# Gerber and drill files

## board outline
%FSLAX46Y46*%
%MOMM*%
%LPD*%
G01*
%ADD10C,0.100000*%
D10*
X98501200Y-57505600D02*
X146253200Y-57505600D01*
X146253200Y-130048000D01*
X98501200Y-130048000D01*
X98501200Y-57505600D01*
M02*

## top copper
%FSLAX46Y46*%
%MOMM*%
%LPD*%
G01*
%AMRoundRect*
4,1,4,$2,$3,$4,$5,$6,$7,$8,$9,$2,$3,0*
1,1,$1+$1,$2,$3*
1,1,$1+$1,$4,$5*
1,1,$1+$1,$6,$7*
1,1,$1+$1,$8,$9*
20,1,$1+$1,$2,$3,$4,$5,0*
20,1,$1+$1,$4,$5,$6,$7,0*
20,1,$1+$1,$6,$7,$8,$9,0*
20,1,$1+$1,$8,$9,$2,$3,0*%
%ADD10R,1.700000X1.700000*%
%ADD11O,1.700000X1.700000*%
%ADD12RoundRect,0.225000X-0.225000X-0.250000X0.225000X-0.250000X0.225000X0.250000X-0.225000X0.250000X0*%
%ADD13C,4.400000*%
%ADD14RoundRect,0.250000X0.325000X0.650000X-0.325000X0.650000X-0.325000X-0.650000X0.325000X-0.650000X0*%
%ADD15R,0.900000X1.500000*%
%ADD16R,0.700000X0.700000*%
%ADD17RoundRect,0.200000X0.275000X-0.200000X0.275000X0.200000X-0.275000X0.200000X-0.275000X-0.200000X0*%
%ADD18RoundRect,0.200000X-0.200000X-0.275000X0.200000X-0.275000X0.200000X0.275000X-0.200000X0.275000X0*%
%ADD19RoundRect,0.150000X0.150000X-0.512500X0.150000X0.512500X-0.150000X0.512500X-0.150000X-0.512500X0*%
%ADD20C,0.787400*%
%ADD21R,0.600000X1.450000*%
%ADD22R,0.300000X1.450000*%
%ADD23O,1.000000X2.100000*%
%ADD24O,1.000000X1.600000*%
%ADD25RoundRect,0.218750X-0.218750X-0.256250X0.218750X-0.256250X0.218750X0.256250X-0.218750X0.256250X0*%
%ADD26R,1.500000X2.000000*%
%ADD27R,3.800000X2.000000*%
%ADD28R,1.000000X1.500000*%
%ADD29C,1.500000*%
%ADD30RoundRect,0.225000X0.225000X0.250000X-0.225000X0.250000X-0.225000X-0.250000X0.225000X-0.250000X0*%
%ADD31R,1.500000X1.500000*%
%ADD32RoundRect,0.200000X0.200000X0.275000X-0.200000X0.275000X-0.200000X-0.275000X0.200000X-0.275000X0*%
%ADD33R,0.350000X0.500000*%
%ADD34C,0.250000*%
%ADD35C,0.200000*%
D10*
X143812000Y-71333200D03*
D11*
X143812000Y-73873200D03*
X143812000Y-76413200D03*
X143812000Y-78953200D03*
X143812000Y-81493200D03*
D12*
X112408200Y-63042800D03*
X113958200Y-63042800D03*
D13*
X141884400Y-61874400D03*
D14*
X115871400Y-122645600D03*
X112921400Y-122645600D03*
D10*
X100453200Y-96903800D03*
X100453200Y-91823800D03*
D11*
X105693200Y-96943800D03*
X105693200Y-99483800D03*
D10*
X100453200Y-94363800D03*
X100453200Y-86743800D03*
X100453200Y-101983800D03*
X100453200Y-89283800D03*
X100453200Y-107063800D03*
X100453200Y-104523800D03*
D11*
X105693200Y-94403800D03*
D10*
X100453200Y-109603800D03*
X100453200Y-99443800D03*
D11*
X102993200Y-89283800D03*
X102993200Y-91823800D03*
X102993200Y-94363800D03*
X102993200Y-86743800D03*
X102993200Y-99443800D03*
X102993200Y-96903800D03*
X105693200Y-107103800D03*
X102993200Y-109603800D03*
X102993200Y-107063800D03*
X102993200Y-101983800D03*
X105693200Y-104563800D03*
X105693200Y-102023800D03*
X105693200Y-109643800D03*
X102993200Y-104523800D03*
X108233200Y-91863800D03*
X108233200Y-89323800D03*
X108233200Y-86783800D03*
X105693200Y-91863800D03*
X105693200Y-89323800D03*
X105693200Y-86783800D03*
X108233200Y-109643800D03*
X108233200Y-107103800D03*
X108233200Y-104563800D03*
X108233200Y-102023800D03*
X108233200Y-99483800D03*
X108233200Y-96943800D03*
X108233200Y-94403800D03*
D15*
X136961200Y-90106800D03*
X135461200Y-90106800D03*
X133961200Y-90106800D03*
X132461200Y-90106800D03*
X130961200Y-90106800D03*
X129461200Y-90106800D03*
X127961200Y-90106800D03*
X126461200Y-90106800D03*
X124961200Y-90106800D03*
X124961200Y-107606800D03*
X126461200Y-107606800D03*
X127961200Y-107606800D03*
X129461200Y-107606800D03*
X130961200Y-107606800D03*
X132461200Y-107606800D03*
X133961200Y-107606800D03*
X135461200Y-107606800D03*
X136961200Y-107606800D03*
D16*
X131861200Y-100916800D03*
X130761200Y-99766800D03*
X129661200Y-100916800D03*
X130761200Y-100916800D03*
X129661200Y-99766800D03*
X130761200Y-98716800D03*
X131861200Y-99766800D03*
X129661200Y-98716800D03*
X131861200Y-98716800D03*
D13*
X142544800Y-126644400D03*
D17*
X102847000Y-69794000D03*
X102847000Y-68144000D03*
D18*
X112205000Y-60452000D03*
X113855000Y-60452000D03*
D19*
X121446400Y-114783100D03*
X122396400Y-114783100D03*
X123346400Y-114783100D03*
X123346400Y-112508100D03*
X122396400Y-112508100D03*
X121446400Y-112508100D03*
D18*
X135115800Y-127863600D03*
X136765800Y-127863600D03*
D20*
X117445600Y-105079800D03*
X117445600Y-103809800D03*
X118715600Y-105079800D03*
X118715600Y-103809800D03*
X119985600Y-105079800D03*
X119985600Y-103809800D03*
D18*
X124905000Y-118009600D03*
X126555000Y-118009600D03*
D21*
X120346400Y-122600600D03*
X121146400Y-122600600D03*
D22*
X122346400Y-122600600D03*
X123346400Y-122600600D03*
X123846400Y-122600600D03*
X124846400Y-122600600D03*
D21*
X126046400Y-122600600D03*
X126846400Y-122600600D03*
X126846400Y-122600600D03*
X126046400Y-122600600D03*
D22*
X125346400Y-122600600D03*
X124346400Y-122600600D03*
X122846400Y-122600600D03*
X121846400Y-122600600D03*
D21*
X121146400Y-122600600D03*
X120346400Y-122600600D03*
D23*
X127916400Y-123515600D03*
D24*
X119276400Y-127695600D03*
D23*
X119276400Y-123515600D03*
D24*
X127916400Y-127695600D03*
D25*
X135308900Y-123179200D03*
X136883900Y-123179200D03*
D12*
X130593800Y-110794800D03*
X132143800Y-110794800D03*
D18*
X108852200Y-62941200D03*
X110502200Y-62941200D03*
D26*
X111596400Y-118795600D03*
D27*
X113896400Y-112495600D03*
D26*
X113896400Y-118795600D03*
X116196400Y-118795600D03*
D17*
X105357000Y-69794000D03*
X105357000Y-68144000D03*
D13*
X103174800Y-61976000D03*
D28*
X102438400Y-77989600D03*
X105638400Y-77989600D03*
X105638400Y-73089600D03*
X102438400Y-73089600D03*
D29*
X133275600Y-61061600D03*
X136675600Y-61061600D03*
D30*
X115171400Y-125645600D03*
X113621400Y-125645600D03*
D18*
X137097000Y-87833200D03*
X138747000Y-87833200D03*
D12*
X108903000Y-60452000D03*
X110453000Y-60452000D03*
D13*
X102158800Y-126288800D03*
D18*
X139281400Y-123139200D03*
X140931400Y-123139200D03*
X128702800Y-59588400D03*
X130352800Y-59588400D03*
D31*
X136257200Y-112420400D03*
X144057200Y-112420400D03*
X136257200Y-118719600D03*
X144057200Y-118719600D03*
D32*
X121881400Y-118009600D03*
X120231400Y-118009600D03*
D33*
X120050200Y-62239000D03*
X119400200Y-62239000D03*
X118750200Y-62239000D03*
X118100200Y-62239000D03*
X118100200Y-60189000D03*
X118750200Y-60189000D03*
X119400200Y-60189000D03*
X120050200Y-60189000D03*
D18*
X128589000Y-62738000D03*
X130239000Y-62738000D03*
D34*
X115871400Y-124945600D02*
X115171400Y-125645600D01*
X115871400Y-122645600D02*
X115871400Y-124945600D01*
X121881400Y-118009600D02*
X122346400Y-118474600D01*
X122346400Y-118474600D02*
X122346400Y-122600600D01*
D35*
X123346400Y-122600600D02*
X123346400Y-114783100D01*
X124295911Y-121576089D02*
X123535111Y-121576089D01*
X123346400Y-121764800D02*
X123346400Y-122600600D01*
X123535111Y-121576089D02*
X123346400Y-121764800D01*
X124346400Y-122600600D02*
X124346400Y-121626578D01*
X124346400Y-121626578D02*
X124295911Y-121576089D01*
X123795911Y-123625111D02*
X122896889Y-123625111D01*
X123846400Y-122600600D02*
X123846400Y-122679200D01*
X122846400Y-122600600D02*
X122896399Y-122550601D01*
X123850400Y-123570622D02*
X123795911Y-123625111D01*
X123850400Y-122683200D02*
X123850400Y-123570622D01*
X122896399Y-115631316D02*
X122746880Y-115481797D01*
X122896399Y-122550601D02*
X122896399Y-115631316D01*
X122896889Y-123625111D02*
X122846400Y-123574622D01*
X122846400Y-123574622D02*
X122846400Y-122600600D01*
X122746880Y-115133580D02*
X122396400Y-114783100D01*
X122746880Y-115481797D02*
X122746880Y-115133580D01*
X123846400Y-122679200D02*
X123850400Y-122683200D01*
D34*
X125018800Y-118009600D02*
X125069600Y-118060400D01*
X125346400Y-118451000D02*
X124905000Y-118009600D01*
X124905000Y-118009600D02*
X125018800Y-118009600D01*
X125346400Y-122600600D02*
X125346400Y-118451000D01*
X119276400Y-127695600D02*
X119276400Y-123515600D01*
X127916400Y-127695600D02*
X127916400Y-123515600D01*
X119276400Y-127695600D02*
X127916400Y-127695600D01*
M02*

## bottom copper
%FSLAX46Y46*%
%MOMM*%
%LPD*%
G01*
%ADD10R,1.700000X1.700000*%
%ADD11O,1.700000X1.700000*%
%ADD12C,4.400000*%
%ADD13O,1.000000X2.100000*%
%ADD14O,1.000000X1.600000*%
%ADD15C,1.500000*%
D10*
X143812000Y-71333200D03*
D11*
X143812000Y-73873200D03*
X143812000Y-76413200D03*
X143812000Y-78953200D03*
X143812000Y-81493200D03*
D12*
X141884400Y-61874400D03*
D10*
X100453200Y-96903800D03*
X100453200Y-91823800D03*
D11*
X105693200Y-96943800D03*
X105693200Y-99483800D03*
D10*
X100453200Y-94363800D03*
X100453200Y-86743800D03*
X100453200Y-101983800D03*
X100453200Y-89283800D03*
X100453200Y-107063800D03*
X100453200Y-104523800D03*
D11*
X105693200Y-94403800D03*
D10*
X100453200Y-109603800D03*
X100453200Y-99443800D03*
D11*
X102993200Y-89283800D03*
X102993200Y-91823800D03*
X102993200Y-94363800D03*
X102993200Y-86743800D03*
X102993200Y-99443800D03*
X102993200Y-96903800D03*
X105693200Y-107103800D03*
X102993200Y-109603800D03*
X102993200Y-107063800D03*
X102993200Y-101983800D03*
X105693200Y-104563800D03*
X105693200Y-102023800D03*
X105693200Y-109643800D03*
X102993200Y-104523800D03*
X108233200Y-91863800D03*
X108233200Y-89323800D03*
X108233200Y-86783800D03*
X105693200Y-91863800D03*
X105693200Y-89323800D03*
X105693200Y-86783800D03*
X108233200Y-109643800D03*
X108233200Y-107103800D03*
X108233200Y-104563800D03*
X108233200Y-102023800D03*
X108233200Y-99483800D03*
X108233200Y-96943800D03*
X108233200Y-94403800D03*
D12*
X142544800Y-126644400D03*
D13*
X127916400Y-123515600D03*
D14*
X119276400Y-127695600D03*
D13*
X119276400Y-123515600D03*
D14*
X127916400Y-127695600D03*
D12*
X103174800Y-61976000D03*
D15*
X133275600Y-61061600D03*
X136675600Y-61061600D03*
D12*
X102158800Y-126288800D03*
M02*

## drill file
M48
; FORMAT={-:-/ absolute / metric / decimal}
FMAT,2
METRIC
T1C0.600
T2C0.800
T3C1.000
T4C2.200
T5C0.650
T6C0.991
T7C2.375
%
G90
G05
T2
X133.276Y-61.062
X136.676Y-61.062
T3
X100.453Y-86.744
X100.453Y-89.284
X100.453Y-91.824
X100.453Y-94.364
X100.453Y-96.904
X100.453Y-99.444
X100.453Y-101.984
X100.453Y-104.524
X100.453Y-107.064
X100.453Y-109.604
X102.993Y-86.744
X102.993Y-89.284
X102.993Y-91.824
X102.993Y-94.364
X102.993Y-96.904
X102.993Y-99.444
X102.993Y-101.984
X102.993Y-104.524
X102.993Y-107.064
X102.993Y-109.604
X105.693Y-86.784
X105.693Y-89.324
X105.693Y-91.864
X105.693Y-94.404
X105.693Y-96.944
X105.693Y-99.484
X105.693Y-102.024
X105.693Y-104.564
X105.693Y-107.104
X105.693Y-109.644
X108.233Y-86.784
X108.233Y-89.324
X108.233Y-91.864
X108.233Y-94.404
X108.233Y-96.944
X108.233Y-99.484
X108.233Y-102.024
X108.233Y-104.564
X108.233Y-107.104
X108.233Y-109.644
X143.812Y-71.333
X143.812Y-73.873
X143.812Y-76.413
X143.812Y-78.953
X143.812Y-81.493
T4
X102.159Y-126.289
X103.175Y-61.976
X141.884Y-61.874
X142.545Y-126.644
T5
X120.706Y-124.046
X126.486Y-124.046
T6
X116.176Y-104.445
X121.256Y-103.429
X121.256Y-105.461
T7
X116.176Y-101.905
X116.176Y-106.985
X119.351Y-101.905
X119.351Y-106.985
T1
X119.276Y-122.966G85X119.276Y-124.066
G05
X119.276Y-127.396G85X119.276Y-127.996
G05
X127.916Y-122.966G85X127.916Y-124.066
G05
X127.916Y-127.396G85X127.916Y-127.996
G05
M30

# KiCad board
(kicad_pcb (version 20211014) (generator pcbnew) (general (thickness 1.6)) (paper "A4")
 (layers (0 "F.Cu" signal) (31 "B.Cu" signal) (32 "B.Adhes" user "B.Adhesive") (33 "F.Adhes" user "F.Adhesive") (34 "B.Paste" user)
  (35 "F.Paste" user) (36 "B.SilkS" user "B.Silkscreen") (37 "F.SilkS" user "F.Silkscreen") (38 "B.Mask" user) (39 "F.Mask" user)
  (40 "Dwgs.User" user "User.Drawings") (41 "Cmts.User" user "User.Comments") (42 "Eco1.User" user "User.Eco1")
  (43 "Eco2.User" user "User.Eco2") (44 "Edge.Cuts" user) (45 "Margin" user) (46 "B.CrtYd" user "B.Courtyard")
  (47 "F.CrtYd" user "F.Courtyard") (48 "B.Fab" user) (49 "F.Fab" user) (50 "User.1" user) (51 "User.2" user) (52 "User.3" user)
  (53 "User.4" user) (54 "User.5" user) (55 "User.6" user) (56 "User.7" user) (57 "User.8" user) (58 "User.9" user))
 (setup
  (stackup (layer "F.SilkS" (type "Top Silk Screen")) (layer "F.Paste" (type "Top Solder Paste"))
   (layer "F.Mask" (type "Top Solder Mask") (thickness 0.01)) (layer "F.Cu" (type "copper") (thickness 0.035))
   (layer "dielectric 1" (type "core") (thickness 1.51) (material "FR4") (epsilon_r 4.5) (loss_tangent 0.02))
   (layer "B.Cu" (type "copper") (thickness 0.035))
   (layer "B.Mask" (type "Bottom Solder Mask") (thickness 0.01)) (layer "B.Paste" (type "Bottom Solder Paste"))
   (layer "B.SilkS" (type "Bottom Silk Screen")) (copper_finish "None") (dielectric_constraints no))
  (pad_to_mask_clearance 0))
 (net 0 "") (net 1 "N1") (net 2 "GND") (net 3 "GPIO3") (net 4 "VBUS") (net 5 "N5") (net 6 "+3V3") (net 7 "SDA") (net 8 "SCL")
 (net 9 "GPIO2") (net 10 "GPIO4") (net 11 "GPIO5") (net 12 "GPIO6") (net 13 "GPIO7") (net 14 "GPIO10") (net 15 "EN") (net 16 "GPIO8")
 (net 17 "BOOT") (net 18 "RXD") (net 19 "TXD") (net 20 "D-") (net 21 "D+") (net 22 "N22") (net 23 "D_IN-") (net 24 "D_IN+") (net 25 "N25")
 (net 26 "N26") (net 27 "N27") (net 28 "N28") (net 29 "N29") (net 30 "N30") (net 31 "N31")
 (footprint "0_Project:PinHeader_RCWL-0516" (layer "F.Cu") (at 143.812 71.3332)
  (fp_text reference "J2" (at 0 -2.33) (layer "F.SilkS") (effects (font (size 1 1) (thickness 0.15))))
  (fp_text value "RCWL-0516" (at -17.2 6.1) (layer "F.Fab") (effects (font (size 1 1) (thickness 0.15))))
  (pad "1" thru_hole rect (at 0 0) (size 1.7 1.7) (drill 1) (layers *.Cu *.Mask) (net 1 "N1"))
  (pad "2" thru_hole oval (at 0 2.54) (size 1.7 1.7) (drill 1) (layers *.Cu *.Mask) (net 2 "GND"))
  (pad "3" thru_hole oval (at 0 5.08) (size 1.7 1.7) (drill 1) (layers *.Cu *.Mask) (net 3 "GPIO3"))
  (pad "4" thru_hole oval (at 0 7.62) (size 1.7 1.7) (drill 1) (layers *.Cu *.Mask) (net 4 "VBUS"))
  (pad "5" thru_hole oval (at 0 10.16) (size 1.7 1.7) (drill 1) (layers *.Cu *.Mask) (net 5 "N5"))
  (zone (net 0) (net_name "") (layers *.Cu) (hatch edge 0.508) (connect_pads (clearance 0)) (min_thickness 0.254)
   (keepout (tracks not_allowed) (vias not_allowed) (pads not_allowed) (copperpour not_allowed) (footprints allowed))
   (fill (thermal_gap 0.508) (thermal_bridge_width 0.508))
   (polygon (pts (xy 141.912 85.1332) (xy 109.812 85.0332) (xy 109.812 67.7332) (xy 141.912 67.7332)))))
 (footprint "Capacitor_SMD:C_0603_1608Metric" (layer "F.Cu") (at 113.1832 63.0428)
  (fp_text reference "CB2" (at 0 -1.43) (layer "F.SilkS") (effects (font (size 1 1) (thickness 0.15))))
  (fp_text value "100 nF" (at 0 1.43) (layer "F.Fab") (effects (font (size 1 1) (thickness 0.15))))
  (pad "1" smd roundrect (at -0.775 0) (size 0.9 0.95) (layers "F.Cu" "F.Paste" "F.Mask") (roundrect_rratio 0.25) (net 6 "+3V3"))
  (pad "2" smd roundrect (at 0.775 0) (size 0.9 0.95) (layers "F.Cu" "F.Paste" "F.Mask") (roundrect_rratio 0.25) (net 2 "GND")))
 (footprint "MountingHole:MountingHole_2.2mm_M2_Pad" (layer "F.Cu") (at 141.8844 61.8744)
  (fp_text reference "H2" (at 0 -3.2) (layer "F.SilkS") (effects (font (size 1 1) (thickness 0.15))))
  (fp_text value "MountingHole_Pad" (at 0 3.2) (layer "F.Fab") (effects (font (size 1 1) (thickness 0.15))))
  (pad "1" thru_hole circle (at 0 0) (size 4.4 4.4) (drill 2.2) (layers *.Cu *.Mask) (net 2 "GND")))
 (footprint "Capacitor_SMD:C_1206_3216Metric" (layer "F.Cu") (at 114.3964 122.6456 180)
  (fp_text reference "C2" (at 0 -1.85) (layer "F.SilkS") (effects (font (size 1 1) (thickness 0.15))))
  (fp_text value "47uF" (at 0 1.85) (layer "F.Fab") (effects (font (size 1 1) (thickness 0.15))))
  (pad "1" smd roundrect (at -1.475 0 180) (size 1.15 1.8) (layers "F.Cu" "F.Paste" "F.Mask") (roundrect_rratio 0.217391) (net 4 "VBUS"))
  (pad "2" smd roundrect (at 1.475 0 180) (size 1.15 1.8) (layers "F.Cu" "F.Paste" "F.Mask") (roundrect_rratio 0.217391) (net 2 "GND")))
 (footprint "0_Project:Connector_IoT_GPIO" (layer "F.Cu") (at 106.8932 114.7038 180)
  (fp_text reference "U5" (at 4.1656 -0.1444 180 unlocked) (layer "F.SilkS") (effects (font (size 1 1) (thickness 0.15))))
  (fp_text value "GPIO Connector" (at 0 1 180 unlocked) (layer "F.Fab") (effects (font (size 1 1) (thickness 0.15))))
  (pad "1" thru_hole rect (at 6.44 17.8 180) (size 1.7 1.7) (drill 1) (layers *.Cu *.Mask) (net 2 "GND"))
  (pad "1" thru_hole rect (at 6.44 22.88 180) (size 1.7 1.7) (drill 1) (layers *.Cu *.Mask) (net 2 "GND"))
  (pad "1" thru_hole oval (at 1.2 17.76 180) (size 1.7 1.7) (drill 1) (layers *.Cu *.Mask) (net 2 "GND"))
  (pad "1" thru_hole oval (at 1.2 15.22 180) (size 1.7 1.7) (drill 1) (layers *.Cu *.Mask) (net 2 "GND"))
  (pad "1" thru_hole rect (at 6.44 20.34 180) (size 1.7 1.7) (drill 1) (layers *.Cu *.Mask) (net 2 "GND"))
  (pad "1" thru_hole rect (at 6.44 27.96 180) (size 1.7 1.7) (drill 1) (layers *.Cu *.Mask) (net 2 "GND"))
  (pad "1" thru_hole rect (at 6.44 12.72 180) (size 1.7 1.7) (drill 1) (layers *.Cu *.Mask) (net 2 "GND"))
  (pad "1" thru_hole rect (at 6.44 25.42 180) (size 1.7 1.7) (drill 1) (layers *.Cu *.Mask) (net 2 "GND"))
  (pad "1" thru_hole rect (at 6.44 7.64 180) (size 1.7 1.7) (drill 1) (layers *.Cu *.Mask) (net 2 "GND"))
  (pad "1" thru_hole rect (at 6.44 10.18 180) (size 1.7 1.7) (drill 1) (layers *.Cu *.Mask) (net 2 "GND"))
  (pad "1" thru_hole oval (at 1.2 20.3 180) (size 1.7 1.7) (drill 1) (layers *.Cu *.Mask) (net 2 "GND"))
  (pad "1" thru_hole rect (at 6.44 5.1 180) (size 1.7 1.7) (drill 1) (layers *.Cu *.Mask) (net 2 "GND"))
  (pad "1" thru_hole rect (at 6.44 15.26 180) (size 1.7 1.7) (drill 1) (layers *.Cu *.Mask) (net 2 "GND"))
  (pad "2" thru_hole oval (at 3.9 25.42 180) (size 1.7 1.7) (drill 1) (layers *.Cu *.Mask) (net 6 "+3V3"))
  (pad "2" thru_hole oval (at 3.9 22.88 180) (size 1.7 1.7) (drill 1) (layers *.Cu *.Mask) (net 6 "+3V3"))
  (pad "2" thru_hole oval (at 3.9 20.34 180) (size 1.7 1.7) (drill 1) (layers *.Cu *.Mask) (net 6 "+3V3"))
  (pad "2" thru_hole oval (at 3.9 27.96 180) (size 1.7 1.7) (drill 1) (layers *.Cu *.Mask) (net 6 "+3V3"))
  (pad "2" thru_hole oval (at 3.9 15.26 180) (size 1.7 1.7) (drill 1) (layers *.Cu *.Mask) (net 6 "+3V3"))
  (pad "2" thru_hole oval (at 3.9 17.8 180) (size 1.7 1.7) (drill 1) (layers *.Cu *.Mask) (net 6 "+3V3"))
  (pad "3" thru_hole oval (at 1.2 7.6 180) (size 1.7 1.7) (drill 1) (layers *.Cu *.Mask) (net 4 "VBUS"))
  (pad "3" thru_hole oval (at 3.9 5.1 180) (size 1.7 1.7) (drill 1) (layers *.Cu *.Mask) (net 4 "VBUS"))
  (pad "3" thru_hole oval (at 3.9 7.64 180) (size 1.7 1.7) (drill 1) (layers *.Cu *.Mask) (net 4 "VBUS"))
  (pad "3" thru_hole oval (at 3.9 12.72 180) (size 1.7 1.7) (drill 1) (layers *.Cu *.Mask) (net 4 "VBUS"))
  (pad "3" thru_hole oval (at 1.2 10.14 180) (size 1.7 1.7) (drill 1) (layers *.Cu *.Mask) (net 4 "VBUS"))
  (pad "3" thru_hole oval (at 1.2 12.68 180) (size 1.7 1.7) (drill 1) (layers *.Cu *.Mask) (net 4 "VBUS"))
  (pad "3" thru_hole oval (at 1.2 5.06 180) (size 1.7 1.7) (drill 1) (layers *.Cu *.Mask) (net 4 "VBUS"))
  (pad "3" thru_hole oval (at 3.9 10.18 180) (size 1.7 1.7) (drill 1) (layers *.Cu *.Mask) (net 4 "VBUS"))
  (pad "4" thru_hole oval (at -1.34 22.84 180) (size 1.7 1.7) (drill 1) (layers *.Cu *.Mask) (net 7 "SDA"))
  (pad "4" thru_hole oval (at -1.34 25.38 180) (size 1.7 1.7) (drill 1) (layers *.Cu *.Mask) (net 7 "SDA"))
  (pad "4" thru_hole oval (at -1.34 27.92 180) (size 1.7 1.7) (drill 1) (layers *.Cu *.Mask) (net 7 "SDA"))
  (pad "5" thru_hole oval (at 1.2 22.84 180) (size 1.7 1.7) (drill 1) (layers *.Cu *.Mask) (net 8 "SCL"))
  (pad "5" thru_hole oval (at 1.2 25.38 180) (size 1.7 1.7) (drill 1) (layers *.Cu *.Mask) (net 8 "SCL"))
  (pad "5" thru_hole oval (at 1.2 27.92 180) (size 1.7 1.7) (drill 1) (layers *.Cu *.Mask) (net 8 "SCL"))
  (pad "6" thru_hole oval (at -1.34 5.06 180) (size 1.7 1.7) (drill 1) (layers *.Cu *.Mask) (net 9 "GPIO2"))
  (pad "7" thru_hole oval (at -1.34 7.6 180) (size 1.7 1.7) (drill 1) (layers *.Cu *.Mask) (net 3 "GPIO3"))
  (pad "8" thru_hole oval (at -1.34 10.14 180) (size 1.7 1.7) (drill 1) (layers *.Cu *.Mask) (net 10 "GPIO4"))
  (pad "9" thru_hole oval (at -1.34 12.68 180) (size 1.7 1.7) (drill 1) (layers *.Cu *.Mask) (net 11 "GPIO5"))
  (pad "10" thru_hole oval (at -1.34 15.22 180) (size 1.7 1.7) (drill 1) (layers *.Cu *.Mask) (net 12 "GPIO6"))
  (pad "11" thru_hole oval (at -1.34 17.76 180) (size 1.7 1.7) (drill 1) (layers *.Cu *.Mask) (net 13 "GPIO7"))
  (pad "12" thru_hole oval (at -1.34 20.3 180) (size 1.7 1.7) (drill 1) (layers *.Cu *.Mask) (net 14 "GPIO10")))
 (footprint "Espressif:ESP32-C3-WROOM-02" (layer "F.Cu") (at 132.8112 98.8568 -90)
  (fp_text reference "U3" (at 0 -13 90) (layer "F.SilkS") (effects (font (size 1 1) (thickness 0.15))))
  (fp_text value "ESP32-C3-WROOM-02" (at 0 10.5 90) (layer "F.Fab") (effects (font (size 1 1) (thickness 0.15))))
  (pad "1" smd rect locked (at -8.75 -4.15 270) (size 1.5 0.9) (layers "F.Cu" "F.Paste" "F.Mask") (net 6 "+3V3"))
  (pad "2" smd rect locked (at -8.75 -2.65 270) (size 1.5 0.9) (layers "F.Cu" "F.Paste" "F.Mask") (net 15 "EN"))
  (pad "3" smd rect locked (at -8.75 -1.15 270) (size 1.5 0.9) (layers "F.Cu" "F.Paste" "F.Mask") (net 10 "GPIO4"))
  (pad "4" smd rect locked (at -8.75 0.35 270) (size 1.5 0.9) (layers "F.Cu" "F.Paste" "F.Mask") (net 11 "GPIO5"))
  (pad "5" smd rect locked (at -8.75 1.85 270) (size 1.5 0.9) (layers "F.Cu" "F.Paste" "F.Mask") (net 12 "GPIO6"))
  (pad "6" smd rect locked (at -8.75 3.35 270) (size 1.5 0.9) (layers "F.Cu" "F.Paste" "F.Mask") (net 13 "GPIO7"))
  (pad "7" smd rect locked (at -8.75 4.85 270) (size 1.5 0.9) (layers "F.Cu" "F.Paste" "F.Mask") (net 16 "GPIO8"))
  (pad "8" smd rect locked (at -8.75 6.35 270) (size 1.5 0.9) (layers "F.Cu" "F.Paste" "F.Mask") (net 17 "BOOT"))
  (pad "9" smd rect locked (at -8.75 7.85 270) (size 1.5 0.9) (layers "F.Cu" "F.Paste" "F.Mask") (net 2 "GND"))
  (pad "10" smd rect locked (at 8.75 7.85 90) (size 1.5 0.9) (layers "F.Cu" "F.Paste" "F.Mask") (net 14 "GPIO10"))
  (pad "11" smd rect locked (at 8.75 6.35 90) (size 1.5 0.9) (layers "F.Cu" "F.Paste" "F.Mask") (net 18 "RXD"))
  (pad "12" smd rect locked (at 8.75 4.85 90) (size 1.5 0.9) (layers "F.Cu" "F.Paste" "F.Mask") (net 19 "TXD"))
  (pad "13" smd rect locked (at 8.75 3.35 90) (size 1.5 0.9) (layers "F.Cu" "F.Paste" "F.Mask") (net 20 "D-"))
  (pad "14" smd rect locked (at 8.75 1.85 90) (size 1.5 0.9) (layers "F.Cu" "F.Paste" "F.Mask") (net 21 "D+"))
  (pad "15" smd rect locked (at 8.75 0.35 90) (size 1.5 0.9) (layers "F.Cu" "F.Paste" "F.Mask") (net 3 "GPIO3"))
  (pad "16" smd rect locked (at 8.75 -1.15 90) (size 1.5 0.9) (layers "F.Cu" "F.Paste" "F.Mask") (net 9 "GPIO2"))
  (pad "17" smd rect locked (at 8.75 -2.65 90) (size 1.5 0.9) (layers "F.Cu" "F.Paste" "F.Mask") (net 8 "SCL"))
  (pad "18" smd rect locked (at 8.75 -4.15 90) (size 1.5 0.9) (layers "F.Cu" "F.Paste" "F.Mask") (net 7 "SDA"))
  (pad "19" smd rect locked (at 2.06 0.95 90) (size 0.7 0.7) (layers "F.Cu" "F.Paste" "F.Mask") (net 2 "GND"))
  (pad "19" smd rect locked (at 0.91 2.05 90) (size 0.7 0.7) (layers "F.Cu" "F.Paste" "F.Mask") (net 2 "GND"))
  (pad "19" smd rect locked (at 2.06 3.15 90) (size 0.7 0.7) (layers "F.Cu" "F.Paste" "F.Mask") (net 2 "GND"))
  (pad "19" smd rect locked (at 2.06 2.05 90) (size 0.7 0.7) (layers "F.Cu" "F.Paste" "F.Mask") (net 2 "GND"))
  (pad "19" smd rect locked (at 0.91 3.15 90) (size 0.7 0.7) (layers "F.Cu" "F.Paste" "F.Mask") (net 2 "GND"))
  (pad "19" smd rect locked (at -0.14 2.05 90) (size 0.7 0.7) (layers "F.Cu" "F.Paste" "F.Mask") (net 2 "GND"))
  (pad "19" smd rect locked (at 0.91 0.95 90) (size 0.7 0.7) (layers "F.Cu" "F.Paste" "F.Mask") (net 2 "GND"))
  (pad "19" smd rect locked (at -0.14 3.15 90) (size 0.7 0.7) (layers "F.Cu" "F.Paste" "F.Mask") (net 2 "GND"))
  (pad "19" smd rect locked (at -0.14 0.95 90) (size 0.7 0.7) (layers "F.Cu" "F.Paste" "F.Mask") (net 2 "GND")))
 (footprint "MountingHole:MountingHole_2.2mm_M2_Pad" (layer "F.Cu") (at 142.5448 126.6444)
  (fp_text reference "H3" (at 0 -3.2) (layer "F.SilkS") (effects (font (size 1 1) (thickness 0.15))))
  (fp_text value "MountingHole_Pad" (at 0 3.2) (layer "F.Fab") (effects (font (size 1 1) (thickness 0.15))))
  (pad "1" thru_hole circle (at 0 0) (size 4.4 4.4) (drill 2.2) (layers *.Cu *.Mask) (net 2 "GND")))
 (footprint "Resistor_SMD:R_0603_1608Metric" (layer "F.Cu") (at 102.847 68.969 90)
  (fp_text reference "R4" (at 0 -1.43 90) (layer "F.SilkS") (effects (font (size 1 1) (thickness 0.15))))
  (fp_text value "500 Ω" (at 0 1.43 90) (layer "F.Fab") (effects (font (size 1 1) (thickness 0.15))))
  (pad "1" smd roundrect (at -0.825 0 90) (size 0.8 0.95) (layers "F.Cu" "F.Paste" "F.Mask") (roundrect_rratio 0.25) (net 16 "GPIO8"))
  (pad "2" smd roundrect (at 0.825 0 90) (size 0.8 0.95) (layers "F.Cu" "F.Paste" "F.Mask") (roundrect_rratio 0.25) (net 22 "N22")))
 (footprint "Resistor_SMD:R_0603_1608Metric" (layer "F.Cu") (at 113.03 60.452)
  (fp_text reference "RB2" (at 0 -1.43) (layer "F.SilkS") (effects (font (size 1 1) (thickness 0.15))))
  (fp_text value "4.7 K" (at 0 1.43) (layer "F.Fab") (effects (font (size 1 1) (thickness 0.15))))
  (pad "1" smd roundrect (at -0.825 0) (size 0.8 0.95) (layers "F.Cu" "F.Paste" "F.Mask") (roundrect_rratio 0.25) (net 8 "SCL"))
  (pad "2" smd roundrect (at 0.825 0) (size 0.8 0.95) (layers "F.Cu" "F.Paste" "F.Mask") (roundrect_rratio 0.25) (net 6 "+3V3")))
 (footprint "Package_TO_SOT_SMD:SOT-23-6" (layer "F.Cu") (at 122.3964 113.6456 90)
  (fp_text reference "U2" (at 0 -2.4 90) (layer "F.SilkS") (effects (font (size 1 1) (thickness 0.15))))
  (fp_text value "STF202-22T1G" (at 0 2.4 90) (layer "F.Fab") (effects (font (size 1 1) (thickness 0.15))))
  (pad "1" smd roundrect (at -1.1375 -0.95 90) (size 1.325 0.6) (layers "F.Cu" "F.Paste" "F.Mask") (roundrect_rratio 0.25) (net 4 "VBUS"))
  (pad "2" smd roundrect (at -1.1375 0 90) (size 1.325 0.6) (layers "F.Cu" "F.Paste" "F.Mask") (roundrect_rratio 0.25) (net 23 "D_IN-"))
  (pad "3" smd roundrect (at -1.1375 0.95 90) (size 1.325 0.6) (layers "F.Cu" "F.Paste" "F.Mask") (roundrect_rratio 0.25) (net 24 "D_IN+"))
  (pad "4" smd roundrect (at 1.1375 0.95 90) (size 1.325 0.6) (layers "F.Cu" "F.Paste" "F.Mask") (roundrect_rratio 0.25) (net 21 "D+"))
  (pad "5" smd roundrect (at 1.1375 0 90) (size 1.325 0.6) (layers "F.Cu" "F.Paste" "F.Mask") (roundrect_rratio 0.25) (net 20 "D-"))
  (pad "6" smd roundrect (at 1.1375 -0.95 90) (size 1.325 0.6) (layers "F.Cu" "F.Paste" "F.Mask") (roundrect_rratio 0.25) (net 2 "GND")))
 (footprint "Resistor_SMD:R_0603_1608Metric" (layer "F.Cu") (at 135.9408 127.8636)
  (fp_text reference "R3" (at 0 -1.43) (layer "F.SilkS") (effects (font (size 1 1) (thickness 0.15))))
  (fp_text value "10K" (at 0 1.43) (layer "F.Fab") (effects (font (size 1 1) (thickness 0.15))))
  (pad "1" smd roundrect (at -0.825 0) (size 0.8 0.95) (layers "F.Cu" "F.Paste" "F.Mask") (roundrect_rratio 0.25) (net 6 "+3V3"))
  (pad "2" smd roundrect (at 0.825 0) (size 0.8 0.95) (layers "F.Cu" "F.Paste" "F.Mask") (roundrect_rratio 0.25) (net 15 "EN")))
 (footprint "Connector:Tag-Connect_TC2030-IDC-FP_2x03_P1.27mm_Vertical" (layer "F.Cu") (at 118.7156 104.4448)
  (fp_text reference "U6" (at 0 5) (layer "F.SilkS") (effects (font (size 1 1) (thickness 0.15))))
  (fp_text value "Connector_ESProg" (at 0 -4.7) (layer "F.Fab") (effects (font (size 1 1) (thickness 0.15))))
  (pad "" np_thru_hole circle (at 2.54 1.016) (size 0.9906 0.9906) (drill 0.9906) (layers *.Cu *.Mask))
  (pad "" np_thru_hole circle (at -2.54 0) (size 0.9906 0.9906) (drill 0.9906) (layers *.Cu *.Mask))
  (pad "" np_thru_hole circle (at -2.54 -2.54) (size 2.3749 2.3749) (drill 2.3749) (layers *.Cu *.Mask))
  (pad "" np_thru_hole circle (at 2.54 -1.016) (size 0.9906 0.9906) (drill 0.9906) (layers *.Cu *.Mask))
  (pad "" np_thru_hole circle (at -2.54 2.54) (size 2.3749 2.3749) (drill 2.3749) (layers *.Cu *.Mask))
  (pad "" np_thru_hole circle (at 0.635 -2.54) (size 2.3749 2.3749) (drill 2.3749) (layers *.Cu *.Mask))
  (pad "" np_thru_hole circle (at 0.635 2.54) (size 2.3749 2.3749) (drill 2.3749) (layers *.Cu *.Mask))
  (pad "1" connect circle (at -1.27 0.635) (size 0.7874 0.7874) (layers "F.Cu" "F.Mask") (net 2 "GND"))
  (pad "2" connect circle (at -1.27 -0.635) (size 0.7874 0.7874) (layers "F.Cu" "F.Mask") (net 17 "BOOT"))
  (pad "3" connect circle (at 0 0.635) (size 0.7874 0.7874) (layers "F.Cu" "F.Mask") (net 6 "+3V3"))
  (pad "4" connect circle (at 0 -0.635) (size 0.7874 0.7874) (layers "F.Cu" "F.Mask") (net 18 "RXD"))
  (pad "5" connect circle (at 1.27 0.635) (size 0.7874 0.7874) (layers "F.Cu" "F.Mask") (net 19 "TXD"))
  (pad "6" connect circle (at 1.27 -0.635) (size 0.7874 0.7874) (layers "F.Cu" "F.Mask") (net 15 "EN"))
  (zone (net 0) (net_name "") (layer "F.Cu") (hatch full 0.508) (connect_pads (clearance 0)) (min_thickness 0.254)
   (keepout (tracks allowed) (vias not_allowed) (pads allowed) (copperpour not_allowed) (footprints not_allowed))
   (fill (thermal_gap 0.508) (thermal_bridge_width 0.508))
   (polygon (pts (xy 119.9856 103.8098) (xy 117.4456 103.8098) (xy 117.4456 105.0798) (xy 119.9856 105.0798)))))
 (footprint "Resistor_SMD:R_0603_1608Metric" (layer "F.Cu") (at 125.73 118.0096)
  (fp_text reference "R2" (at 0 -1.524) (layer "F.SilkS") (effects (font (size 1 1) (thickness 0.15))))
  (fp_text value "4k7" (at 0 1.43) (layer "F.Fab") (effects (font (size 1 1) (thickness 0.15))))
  (pad "1" smd roundrect (at -0.825 0) (size 0.8 0.95) (layers "F.Cu" "F.Paste" "F.Mask") (roundrect_rratio 0.25) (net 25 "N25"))
  (pad "2" smd roundrect (at 0.825 0) (size 0.8 0.95) (layers "F.Cu" "F.Paste" "F.Mask") (roundrect_rratio 0.25) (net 2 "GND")))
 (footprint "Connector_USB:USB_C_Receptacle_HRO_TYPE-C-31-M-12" (layer "F.Cu") (at 123.5964 126.6456)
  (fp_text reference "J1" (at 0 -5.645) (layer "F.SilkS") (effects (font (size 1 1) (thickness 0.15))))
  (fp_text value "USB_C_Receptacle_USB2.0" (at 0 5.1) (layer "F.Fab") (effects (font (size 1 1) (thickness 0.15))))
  (pad "" np_thru_hole circle (at 2.89 -2.6) (size 0.65 0.65) (drill 0.65) (layers *.Cu *.Mask))
  (pad "" np_thru_hole circle (at -2.89 -2.6) (size 0.65 0.65) (drill 0.65) (layers *.Cu *.Mask))
  (pad "A1" smd rect (at -3.25 -4.045) (size 0.6 1.45) (layers "F.Cu" "F.Paste" "F.Mask") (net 2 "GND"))
  (pad "A4" smd rect (at -2.45 -4.045) (size 0.6 1.45) (layers "F.Cu" "F.Paste" "F.Mask") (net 4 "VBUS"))
  (pad "A5" smd rect (at -1.25 -4.045) (size 0.3 1.45) (layers "F.Cu" "F.Paste" "F.Mask") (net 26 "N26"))
  (pad "A6" smd rect (at -0.25 -4.045) (size 0.3 1.45) (layers "F.Cu" "F.Paste" "F.Mask") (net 24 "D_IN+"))
  (pad "A7" smd rect (at 0.25 -4.045) (size 0.3 1.45) (layers "F.Cu" "F.Paste" "F.Mask") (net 23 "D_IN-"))
  (pad "A8" smd rect (at 1.25 -4.045) (size 0.3 1.45) (layers "F.Cu" "F.Paste" "F.Mask") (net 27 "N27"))
  (pad "A9" smd rect (at 2.45 -4.045) (size 0.6 1.45) (layers "F.Cu" "F.Paste" "F.Mask") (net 4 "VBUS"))
  (pad "A12" smd rect (at 3.25 -4.045) (size 0.6 1.45) (layers "F.Cu" "F.Paste" "F.Mask") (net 2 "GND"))
  (pad "B1" smd rect (at 3.25 -4.045) (size 0.6 1.45) (layers "F.Cu" "F.Paste" "F.Mask") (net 2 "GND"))
  (pad "B4" smd rect (at 2.45 -4.045) (size 0.6 1.45) (layers "F.Cu" "F.Paste" "F.Mask") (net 4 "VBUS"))
  (pad "B5" smd rect (at 1.75 -4.045) (size 0.3 1.45) (layers "F.Cu" "F.Paste" "F.Mask") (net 25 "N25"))
  (pad "B6" smd rect (at 0.75 -4.045) (size 0.3 1.45) (layers "F.Cu" "F.Paste" "F.Mask") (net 24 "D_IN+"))
  (pad "B7" smd rect (at -0.75 -4.045) (size 0.3 1.45) (layers "F.Cu" "F.Paste" "F.Mask") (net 23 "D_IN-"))
  (pad "B8" smd rect (at -1.75 -4.045) (size 0.3 1.45) (layers "F.Cu" "F.Paste" "F.Mask") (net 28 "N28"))
  (pad "B9" smd rect (at -2.45 -4.045) (size 0.6 1.45) (layers "F.Cu" "F.Paste" "F.Mask") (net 4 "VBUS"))
  (pad "B12" smd rect (at -3.25 -4.045) (size 0.6 1.45) (layers "F.Cu" "F.Paste" "F.Mask") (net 2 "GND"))
  (pad "S1" thru_hole oval (at 4.32 -3.13) (size 1 2.1) (drill oval 0.6 1.7) (layers *.Cu *.Mask) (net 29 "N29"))
  (pad "S1" thru_hole oval (at -4.32 1.05) (size 1 1.6) (drill oval 0.6 1.2) (layers *.Cu *.Mask) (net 29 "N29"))
  (pad "S1" thru_hole oval (at -4.32 -3.13) (size 1 2.1) (drill oval 0.6 1.7) (layers *.Cu *.Mask) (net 29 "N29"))
  (pad "S1" thru_hole oval (at 4.32 1.05) (size 1 1.6) (drill oval 0.6 1.2) (layers *.Cu *.Mask) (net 29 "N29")))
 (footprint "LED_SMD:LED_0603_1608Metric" (layer "F.Cu") (at 136.0964 123.1792)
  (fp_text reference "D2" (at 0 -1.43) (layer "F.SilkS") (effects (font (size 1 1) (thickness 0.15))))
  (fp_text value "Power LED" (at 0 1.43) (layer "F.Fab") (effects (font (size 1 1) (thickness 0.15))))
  (pad "1" smd roundrect (at -0.7875 0) (size 0.875 0.95) (layers "F.Cu" "F.Paste" "F.Mask") (roundrect_rratio 0.25) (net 2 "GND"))
  (pad "2" smd roundrect (at 0.7875 0) (size 0.875 0.95) (layers "F.Cu" "F.Paste" "F.Mask") (roundrect_rratio 0.25) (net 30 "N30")))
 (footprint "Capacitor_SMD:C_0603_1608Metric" (layer "F.Cu") (at 131.3688 110.7948)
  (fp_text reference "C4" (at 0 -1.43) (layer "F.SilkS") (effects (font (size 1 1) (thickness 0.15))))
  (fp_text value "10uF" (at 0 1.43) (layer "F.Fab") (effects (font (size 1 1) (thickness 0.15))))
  (pad "1" smd roundrect (at -0.775 0) (size 0.9 0.95) (layers "F.Cu" "F.Paste" "F.Mask") (roundrect_rratio 0.25) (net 6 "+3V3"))
  (pad "2" smd roundrect (at 0.775 0) (size 0.9 0.95) (layers "F.Cu" "F.Paste" "F.Mask") (roundrect_rratio 0.25) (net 2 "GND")))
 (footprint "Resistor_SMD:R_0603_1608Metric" (layer "F.Cu") (at 109.6772 62.9412)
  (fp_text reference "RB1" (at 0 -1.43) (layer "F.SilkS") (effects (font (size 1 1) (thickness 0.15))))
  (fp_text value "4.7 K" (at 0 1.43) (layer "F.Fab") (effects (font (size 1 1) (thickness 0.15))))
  (pad "1" smd roundrect (at -0.825 0) (size 0.8 0.95) (layers "F.Cu" "F.Paste" "F.Mask") (roundrect_rratio 0.25) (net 7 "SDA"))
  (pad "2" smd roundrect (at 0.825 0) (size 0.8 0.95) (layers "F.Cu" "F.Paste" "F.Mask") (roundrect_rratio 0.25) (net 6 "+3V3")))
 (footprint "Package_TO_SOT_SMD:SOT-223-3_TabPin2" (layer "F.Cu") (at 113.8964 115.6456 90)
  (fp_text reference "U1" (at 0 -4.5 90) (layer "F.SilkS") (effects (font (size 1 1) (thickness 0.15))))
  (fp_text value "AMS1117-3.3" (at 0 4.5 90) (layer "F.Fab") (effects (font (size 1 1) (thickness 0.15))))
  (pad "1" smd rect (at -3.15 -2.3 90) (size 2 1.5) (layers "F.Cu" "F.Paste" "F.Mask") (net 2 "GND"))
  (pad "2" smd rect (at 3.15 0 90) (size 2 3.8) (layers "F.Cu" "F.Paste" "F.Mask") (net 6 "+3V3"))
  (pad "2" smd rect (at -3.15 0 90) (size 2 1.5) (layers "F.Cu" "F.Paste" "F.Mask") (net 6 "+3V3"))
  (pad "3" smd rect (at -3.15 2.3 90) (size 2 1.5) (layers "F.Cu" "F.Paste" "F.Mask") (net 4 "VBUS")))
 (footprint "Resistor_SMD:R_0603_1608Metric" (layer "F.Cu") (at 105.357 68.969 90)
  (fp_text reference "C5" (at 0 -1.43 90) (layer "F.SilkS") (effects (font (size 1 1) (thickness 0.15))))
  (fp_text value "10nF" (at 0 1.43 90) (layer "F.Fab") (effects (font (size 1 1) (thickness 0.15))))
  (pad "1" smd roundrect (at -0.825 0 90) (size 0.8 0.95) (layers "F.Cu" "F.Paste" "F.Mask") (roundrect_rratio 0.25) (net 6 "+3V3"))
  (pad "2" smd roundrect (at 0.825 0 90) (size 0.8 0.95) (layers "F.Cu" "F.Paste" "F.Mask") (roundrect_rratio 0.25) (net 2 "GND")))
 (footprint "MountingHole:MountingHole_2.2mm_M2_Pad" (layer "F.Cu") (at 103.1748 61.976)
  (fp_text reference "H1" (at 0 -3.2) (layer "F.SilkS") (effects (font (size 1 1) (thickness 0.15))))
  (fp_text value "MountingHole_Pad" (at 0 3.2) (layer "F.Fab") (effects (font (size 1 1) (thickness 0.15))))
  (pad "1" thru_hole circle (at 0 0) (size 4.4 4.4) (drill 2.2) (layers *.Cu *.Mask) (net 2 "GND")))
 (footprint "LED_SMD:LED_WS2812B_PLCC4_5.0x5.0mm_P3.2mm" (layer "F.Cu") (at 104.0384 75.5396 90)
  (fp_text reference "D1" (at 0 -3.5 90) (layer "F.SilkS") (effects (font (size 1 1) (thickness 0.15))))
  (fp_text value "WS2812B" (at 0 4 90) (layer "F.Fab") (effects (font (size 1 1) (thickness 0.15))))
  (pad "1" smd rect (at -2.45 -1.6 90) (size 1.5 1) (layers "F.Cu" "F.Paste" "F.Mask") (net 6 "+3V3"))
  (pad "2" smd rect (at -2.45 1.6 90) (size 1.5 1) (layers "F.Cu" "F.Paste" "F.Mask") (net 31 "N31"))
  (pad "3" smd rect (at 2.45 1.6 90) (size 1.5 1) (layers "F.Cu" "F.Paste" "F.Mask") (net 2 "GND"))
  (pad "4" smd rect (at 2.45 -1.6 90) (size 1.5 1) (layers "F.Cu" "F.Paste" "F.Mask") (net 22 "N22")))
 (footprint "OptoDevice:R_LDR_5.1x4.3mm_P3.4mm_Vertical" (layer "F.Cu") (at 133.2756 61.0616)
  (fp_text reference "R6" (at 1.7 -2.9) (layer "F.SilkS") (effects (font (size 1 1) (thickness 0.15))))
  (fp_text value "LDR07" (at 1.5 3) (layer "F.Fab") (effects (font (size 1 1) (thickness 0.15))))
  (pad "1" thru_hole circle (at 0 0) (size 1.5 1.5) (drill 0.8) (layers *.Cu *.Mask) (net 6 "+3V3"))
  (pad "2" thru_hole circle (at 3.4 0) (size 1.5 1.5) (drill 0.8) (layers *.Cu *.Mask) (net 9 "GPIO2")))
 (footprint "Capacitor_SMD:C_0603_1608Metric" (layer "F.Cu") (at 114.3964 125.6456 180)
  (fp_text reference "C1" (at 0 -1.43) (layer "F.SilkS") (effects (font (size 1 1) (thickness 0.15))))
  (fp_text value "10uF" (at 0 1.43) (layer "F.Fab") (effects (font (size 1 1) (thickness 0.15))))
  (pad "1" smd roundrect (at -0.775 0 180) (size 0.9 0.95) (layers "F.Cu" "F.Paste" "F.Mask") (roundrect_rratio 0.25) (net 4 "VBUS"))
  (pad "2" smd roundrect (at 0.775 0 180) (size 0.9 0.95) (layers "F.Cu" "F.Paste" "F.Mask") (roundrect_rratio 0.25) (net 2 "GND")))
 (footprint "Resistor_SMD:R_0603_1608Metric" (layer "F.Cu") (at 137.922 87.8332)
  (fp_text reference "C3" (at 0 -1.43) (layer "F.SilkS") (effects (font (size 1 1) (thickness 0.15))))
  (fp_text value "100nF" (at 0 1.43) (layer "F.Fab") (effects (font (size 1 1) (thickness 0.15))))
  (pad "1" smd roundrect (at -0.825 0) (size 0.8 0.95) (layers "F.Cu" "F.Paste" "F.Mask") (roundrect_rratio 0.25) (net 15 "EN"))
  (pad "2" smd roundrect (at 0.825 0) (size 0.8 0.95) (layers "F.Cu" "F.Paste" "F.Mask") (roundrect_rratio 0.25) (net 2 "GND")))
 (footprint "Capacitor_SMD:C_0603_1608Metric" (layer "F.Cu") (at 109.678 60.452)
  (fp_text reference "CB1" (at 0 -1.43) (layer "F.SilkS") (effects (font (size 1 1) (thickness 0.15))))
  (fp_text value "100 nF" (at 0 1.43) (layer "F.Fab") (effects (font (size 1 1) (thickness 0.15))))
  (pad "1" smd roundrect (at -0.775 0) (size 0.9 0.95) (layers "F.Cu" "F.Paste" "F.Mask") (roundrect_rratio 0.25) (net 6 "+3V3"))
  (pad "2" smd roundrect (at 0.775 0) (size 0.9 0.95) (layers "F.Cu" "F.Paste" "F.Mask") (roundrect_rratio 0.25) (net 2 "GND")))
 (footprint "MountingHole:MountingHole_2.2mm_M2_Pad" (layer "F.Cu") (at 102.1588 126.2888)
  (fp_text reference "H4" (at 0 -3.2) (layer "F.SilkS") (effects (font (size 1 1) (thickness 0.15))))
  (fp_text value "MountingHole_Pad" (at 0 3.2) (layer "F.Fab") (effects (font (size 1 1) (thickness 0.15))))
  (pad "1" thru_hole circle (at 0 0) (size 4.4 4.4) (drill 2.2) (layers *.Cu *.Mask) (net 2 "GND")))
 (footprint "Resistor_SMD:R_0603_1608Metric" (layer "F.Cu") (at 140.1064 123.1392)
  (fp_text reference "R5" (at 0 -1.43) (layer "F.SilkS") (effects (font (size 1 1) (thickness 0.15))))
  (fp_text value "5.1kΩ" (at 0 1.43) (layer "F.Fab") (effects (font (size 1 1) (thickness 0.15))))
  (pad "1" smd roundrect (at -0.825 0) (size 0.8 0.95) (layers "F.Cu" "F.Paste" "F.Mask") (roundrect_rratio 0.25) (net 6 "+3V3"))
  (pad "2" smd roundrect (at 0.825 0) (size 0.8 0.95) (layers "F.Cu" "F.Paste" "F.Mask") (roundrect_rratio 0.25) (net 30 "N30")))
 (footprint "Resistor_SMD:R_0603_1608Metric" (layer "F.Cu") (at 129.5278 59.5884)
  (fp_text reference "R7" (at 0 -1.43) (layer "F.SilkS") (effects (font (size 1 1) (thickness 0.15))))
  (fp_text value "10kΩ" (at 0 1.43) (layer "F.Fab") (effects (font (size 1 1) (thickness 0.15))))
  (pad "1" smd roundrect (at -0.825 0) (size 0.8 0.95) (layers "F.Cu" "F.Paste" "F.Mask") (roundrect_rratio 0.25) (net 9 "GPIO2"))
  (pad "2" smd roundrect (at 0.825 0) (size 0.8 0.95) (layers "F.Cu" "F.Paste" "F.Mask") (roundrect_rratio 0.25) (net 2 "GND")))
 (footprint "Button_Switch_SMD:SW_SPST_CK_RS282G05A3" (layer "F.Cu") (at 140.1572 112.4204)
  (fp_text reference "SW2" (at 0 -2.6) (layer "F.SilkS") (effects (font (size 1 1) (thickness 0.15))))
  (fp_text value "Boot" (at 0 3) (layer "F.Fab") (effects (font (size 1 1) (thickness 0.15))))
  (pad "1" smd rect (at -3.9 0) (size 1.5 1.5) (layers "F.Cu" "F.Paste" "F.Mask") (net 2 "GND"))
  (pad "2" smd rect (at 3.9 0) (size 1.5 1.5) (layers "F.Cu" "F.Paste" "F.Mask") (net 17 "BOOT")))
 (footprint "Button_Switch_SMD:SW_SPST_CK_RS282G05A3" (layer "F.Cu") (at 140.1572 118.7196)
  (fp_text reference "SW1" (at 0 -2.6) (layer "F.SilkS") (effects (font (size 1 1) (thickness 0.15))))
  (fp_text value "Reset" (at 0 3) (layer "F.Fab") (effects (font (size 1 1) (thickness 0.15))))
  (pad "1" smd rect (at -3.9 0) (size 1.5 1.5) (layers "F.Cu" "F.Paste" "F.Mask") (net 2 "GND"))
  (pad "2" smd rect (at 3.9 0) (size 1.5 1.5) (layers "F.Cu" "F.Paste" "F.Mask") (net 15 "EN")))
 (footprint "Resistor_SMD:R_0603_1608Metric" (layer "F.Cu") (at 121.0564 118.0096 180)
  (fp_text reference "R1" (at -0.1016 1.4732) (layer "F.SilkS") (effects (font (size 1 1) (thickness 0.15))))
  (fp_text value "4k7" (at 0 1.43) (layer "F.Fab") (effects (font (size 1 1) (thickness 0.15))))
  (pad "1" smd roundrect (at -0.825 0 180) (size 0.8 0.95) (layers "F.Cu" "F.Paste" "F.Mask") (roundrect_rratio 0.25) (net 26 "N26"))
  (pad "2" smd roundrect (at 0.825 0 180) (size 0.8 0.95) (layers "F.Cu" "F.Paste" "F.Mask") (roundrect_rratio 0.25) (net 2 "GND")))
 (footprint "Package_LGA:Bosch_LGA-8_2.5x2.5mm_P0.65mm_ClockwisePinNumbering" (layer "F.Cu") (at 119.0752 61.214 180)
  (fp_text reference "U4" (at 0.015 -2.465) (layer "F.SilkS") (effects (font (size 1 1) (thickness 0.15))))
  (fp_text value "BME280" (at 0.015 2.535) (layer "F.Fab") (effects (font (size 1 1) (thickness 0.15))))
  (pad "1" smd rect (at -0.975 -1.025 270) (size 0.5 0.35) (layers "F.Cu" "F.Paste" "F.Mask") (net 2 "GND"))
  (pad "2" smd rect (at -0.325 -1.025 270) (size 0.5 0.35) (layers "F.Cu" "F.Paste" "F.Mask") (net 6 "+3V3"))
  (pad "3" smd rect (at 0.325 -1.025 270) (size 0.5 0.35) (layers "F.Cu" "F.Paste" "F.Mask") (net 7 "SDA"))
  (pad "4" smd rect (at 0.975 -1.025 270) (size 0.5 0.35) (layers "F.Cu" "F.Paste" "F.Mask") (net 8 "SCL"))
  (pad "5" smd rect (at 0.975 1.025 270) (size 0.5 0.35) (layers "F.Cu" "F.Paste" "F.Mask") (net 6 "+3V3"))
  (pad "6" smd rect (at 0.325 1.025 270) (size 0.5 0.35) (layers "F.Cu" "F.Paste" "F.Mask") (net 6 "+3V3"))
  (pad "7" smd rect (at -0.325 1.025 270) (size 0.5 0.35) (layers "F.Cu" "F.Paste" "F.Mask") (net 2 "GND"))
  (pad "8" smd rect (at -0.975 1.025 270) (size 0.5 0.35) (layers "F.Cu" "F.Paste" "F.Mask") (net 6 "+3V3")))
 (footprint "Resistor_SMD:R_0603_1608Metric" (layer "F.Cu") (at 129.414 62.738)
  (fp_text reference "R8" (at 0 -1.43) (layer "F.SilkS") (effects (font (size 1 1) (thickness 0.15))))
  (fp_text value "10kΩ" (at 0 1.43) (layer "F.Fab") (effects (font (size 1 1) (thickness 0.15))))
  (pad "1" smd roundrect (at -0.825 0) (size 0.8 0.95) (layers "F.Cu" "F.Paste" "F.Mask") (roundrect_rratio 0.25) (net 9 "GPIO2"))
  (pad "2" smd roundrect (at 0.825 0) (size 0.8 0.95) (layers "F.Cu" "F.Paste" "F.Mask") (roundrect_rratio 0.25) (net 6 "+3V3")))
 (gr_rect (start 146.2532 130.048) (end 98.5012 57.5056) (layer "Edge.Cuts") (width 0.1) (fill none))
 (segment (start 115.8714 124.9456) (end 115.1714 125.6456) (width 0.25) (layer "F.Cu") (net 4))
 (segment (start 115.8714 122.6456) (end 115.8714 124.9456) (width 0.25) (layer "F.Cu") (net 4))
 (segment (start 121.8814 118.0096) (end 122.3464 118.4746) (width 0.25) (layer "F.Cu") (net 26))
 (segment (start 122.3464 118.4746) (end 122.3464 122.6006) (width 0.25) (layer "F.Cu") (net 26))
 (segment (start 123.3464 122.6006) (end 123.3464 114.7831) (width 0.2) (layer "F.Cu") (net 24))
 (segment (start 124.295911 121.576089) (end 123.535111 121.576089) (width 0.2) (layer "F.Cu") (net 24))
 (segment (start 123.3464 121.7648) (end 123.3464 122.6006) (width 0.2) (layer "F.Cu") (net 24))
 (segment (start 123.535111 121.576089) (end 123.3464 121.7648) (width 0.2) (layer "F.Cu") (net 24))
 (segment (start 124.3464 122.6006) (end 124.3464 121.626578) (width 0.2) (layer "F.Cu") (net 24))
 (segment (start 124.3464 121.626578) (end 124.295911 121.576089) (width 0.2) (layer "F.Cu") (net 24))
 (segment (start 123.795911 123.625111) (end 122.896889 123.625111) (width 0.2) (layer "F.Cu") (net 23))
 (segment (start 123.8464 122.6006) (end 123.8464 122.6792) (width 0.2) (layer "F.Cu") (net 23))
 (segment (start 122.8464 122.6006) (end 122.896399 122.550601) (width 0.2) (layer "F.Cu") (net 23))
 (segment (start 123.8504 123.570622) (end 123.795911 123.625111) (width 0.2) (layer "F.Cu") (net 23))
 (segment (start 123.8504 122.6832) (end 123.8504 123.570622) (width 0.2) (layer "F.Cu") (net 23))
 (segment (start 122.896399 115.631316) (end 122.74688 115.481797) (width 0.2) (layer "F.Cu") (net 23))
 (segment (start 122.896399 122.550601) (end 122.896399 115.631316) (width 0.2) (layer "F.Cu") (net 23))
 (segment (start 122.896889 123.625111) (end 122.8464 123.574622) (width 0.2) (layer "F.Cu") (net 23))
 (segment (start 122.8464 123.574622) (end 122.8464 122.6006) (width 0.2) (layer "F.Cu") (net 23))
 (segment (start 122.74688 115.13358) (end 122.3964 114.7831) (width 0.2) (layer "F.Cu") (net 23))
 (segment (start 122.74688 115.481797) (end 122.74688 115.13358) (width 0.2) (layer "F.Cu") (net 23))
 (segment (start 123.8464 122.6792) (end 123.8504 122.6832) (width 0.2) (layer "F.Cu") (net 23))
 (segment (start 125.0188 118.0096) (end 125.0696 118.0604) (width 0.25) (layer "F.Cu") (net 25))
 (segment (start 125.3464 118.451) (end 124.905 118.0096) (width 0.25) (layer "F.Cu") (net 25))
 (segment (start 124.905 118.0096) (end 125.0188 118.0096) (width 0.25) (layer "F.Cu") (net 25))
 (segment (start 125.3464 122.6006) (end 125.3464 118.451) (width 0.25) (layer "F.Cu") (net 25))
 (segment (start 119.2764 127.6956) (end 119.2764 123.5156) (width 0.25) (layer "F.Cu") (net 29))
 (segment (start 127.9164 127.6956) (end 127.9164 123.5156) (width 0.25) (layer "F.Cu") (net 29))
 (segment (start 119.2764 127.6956) (end 127.9164 127.6956) (width 0.25) (layer "F.Cu") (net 29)))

